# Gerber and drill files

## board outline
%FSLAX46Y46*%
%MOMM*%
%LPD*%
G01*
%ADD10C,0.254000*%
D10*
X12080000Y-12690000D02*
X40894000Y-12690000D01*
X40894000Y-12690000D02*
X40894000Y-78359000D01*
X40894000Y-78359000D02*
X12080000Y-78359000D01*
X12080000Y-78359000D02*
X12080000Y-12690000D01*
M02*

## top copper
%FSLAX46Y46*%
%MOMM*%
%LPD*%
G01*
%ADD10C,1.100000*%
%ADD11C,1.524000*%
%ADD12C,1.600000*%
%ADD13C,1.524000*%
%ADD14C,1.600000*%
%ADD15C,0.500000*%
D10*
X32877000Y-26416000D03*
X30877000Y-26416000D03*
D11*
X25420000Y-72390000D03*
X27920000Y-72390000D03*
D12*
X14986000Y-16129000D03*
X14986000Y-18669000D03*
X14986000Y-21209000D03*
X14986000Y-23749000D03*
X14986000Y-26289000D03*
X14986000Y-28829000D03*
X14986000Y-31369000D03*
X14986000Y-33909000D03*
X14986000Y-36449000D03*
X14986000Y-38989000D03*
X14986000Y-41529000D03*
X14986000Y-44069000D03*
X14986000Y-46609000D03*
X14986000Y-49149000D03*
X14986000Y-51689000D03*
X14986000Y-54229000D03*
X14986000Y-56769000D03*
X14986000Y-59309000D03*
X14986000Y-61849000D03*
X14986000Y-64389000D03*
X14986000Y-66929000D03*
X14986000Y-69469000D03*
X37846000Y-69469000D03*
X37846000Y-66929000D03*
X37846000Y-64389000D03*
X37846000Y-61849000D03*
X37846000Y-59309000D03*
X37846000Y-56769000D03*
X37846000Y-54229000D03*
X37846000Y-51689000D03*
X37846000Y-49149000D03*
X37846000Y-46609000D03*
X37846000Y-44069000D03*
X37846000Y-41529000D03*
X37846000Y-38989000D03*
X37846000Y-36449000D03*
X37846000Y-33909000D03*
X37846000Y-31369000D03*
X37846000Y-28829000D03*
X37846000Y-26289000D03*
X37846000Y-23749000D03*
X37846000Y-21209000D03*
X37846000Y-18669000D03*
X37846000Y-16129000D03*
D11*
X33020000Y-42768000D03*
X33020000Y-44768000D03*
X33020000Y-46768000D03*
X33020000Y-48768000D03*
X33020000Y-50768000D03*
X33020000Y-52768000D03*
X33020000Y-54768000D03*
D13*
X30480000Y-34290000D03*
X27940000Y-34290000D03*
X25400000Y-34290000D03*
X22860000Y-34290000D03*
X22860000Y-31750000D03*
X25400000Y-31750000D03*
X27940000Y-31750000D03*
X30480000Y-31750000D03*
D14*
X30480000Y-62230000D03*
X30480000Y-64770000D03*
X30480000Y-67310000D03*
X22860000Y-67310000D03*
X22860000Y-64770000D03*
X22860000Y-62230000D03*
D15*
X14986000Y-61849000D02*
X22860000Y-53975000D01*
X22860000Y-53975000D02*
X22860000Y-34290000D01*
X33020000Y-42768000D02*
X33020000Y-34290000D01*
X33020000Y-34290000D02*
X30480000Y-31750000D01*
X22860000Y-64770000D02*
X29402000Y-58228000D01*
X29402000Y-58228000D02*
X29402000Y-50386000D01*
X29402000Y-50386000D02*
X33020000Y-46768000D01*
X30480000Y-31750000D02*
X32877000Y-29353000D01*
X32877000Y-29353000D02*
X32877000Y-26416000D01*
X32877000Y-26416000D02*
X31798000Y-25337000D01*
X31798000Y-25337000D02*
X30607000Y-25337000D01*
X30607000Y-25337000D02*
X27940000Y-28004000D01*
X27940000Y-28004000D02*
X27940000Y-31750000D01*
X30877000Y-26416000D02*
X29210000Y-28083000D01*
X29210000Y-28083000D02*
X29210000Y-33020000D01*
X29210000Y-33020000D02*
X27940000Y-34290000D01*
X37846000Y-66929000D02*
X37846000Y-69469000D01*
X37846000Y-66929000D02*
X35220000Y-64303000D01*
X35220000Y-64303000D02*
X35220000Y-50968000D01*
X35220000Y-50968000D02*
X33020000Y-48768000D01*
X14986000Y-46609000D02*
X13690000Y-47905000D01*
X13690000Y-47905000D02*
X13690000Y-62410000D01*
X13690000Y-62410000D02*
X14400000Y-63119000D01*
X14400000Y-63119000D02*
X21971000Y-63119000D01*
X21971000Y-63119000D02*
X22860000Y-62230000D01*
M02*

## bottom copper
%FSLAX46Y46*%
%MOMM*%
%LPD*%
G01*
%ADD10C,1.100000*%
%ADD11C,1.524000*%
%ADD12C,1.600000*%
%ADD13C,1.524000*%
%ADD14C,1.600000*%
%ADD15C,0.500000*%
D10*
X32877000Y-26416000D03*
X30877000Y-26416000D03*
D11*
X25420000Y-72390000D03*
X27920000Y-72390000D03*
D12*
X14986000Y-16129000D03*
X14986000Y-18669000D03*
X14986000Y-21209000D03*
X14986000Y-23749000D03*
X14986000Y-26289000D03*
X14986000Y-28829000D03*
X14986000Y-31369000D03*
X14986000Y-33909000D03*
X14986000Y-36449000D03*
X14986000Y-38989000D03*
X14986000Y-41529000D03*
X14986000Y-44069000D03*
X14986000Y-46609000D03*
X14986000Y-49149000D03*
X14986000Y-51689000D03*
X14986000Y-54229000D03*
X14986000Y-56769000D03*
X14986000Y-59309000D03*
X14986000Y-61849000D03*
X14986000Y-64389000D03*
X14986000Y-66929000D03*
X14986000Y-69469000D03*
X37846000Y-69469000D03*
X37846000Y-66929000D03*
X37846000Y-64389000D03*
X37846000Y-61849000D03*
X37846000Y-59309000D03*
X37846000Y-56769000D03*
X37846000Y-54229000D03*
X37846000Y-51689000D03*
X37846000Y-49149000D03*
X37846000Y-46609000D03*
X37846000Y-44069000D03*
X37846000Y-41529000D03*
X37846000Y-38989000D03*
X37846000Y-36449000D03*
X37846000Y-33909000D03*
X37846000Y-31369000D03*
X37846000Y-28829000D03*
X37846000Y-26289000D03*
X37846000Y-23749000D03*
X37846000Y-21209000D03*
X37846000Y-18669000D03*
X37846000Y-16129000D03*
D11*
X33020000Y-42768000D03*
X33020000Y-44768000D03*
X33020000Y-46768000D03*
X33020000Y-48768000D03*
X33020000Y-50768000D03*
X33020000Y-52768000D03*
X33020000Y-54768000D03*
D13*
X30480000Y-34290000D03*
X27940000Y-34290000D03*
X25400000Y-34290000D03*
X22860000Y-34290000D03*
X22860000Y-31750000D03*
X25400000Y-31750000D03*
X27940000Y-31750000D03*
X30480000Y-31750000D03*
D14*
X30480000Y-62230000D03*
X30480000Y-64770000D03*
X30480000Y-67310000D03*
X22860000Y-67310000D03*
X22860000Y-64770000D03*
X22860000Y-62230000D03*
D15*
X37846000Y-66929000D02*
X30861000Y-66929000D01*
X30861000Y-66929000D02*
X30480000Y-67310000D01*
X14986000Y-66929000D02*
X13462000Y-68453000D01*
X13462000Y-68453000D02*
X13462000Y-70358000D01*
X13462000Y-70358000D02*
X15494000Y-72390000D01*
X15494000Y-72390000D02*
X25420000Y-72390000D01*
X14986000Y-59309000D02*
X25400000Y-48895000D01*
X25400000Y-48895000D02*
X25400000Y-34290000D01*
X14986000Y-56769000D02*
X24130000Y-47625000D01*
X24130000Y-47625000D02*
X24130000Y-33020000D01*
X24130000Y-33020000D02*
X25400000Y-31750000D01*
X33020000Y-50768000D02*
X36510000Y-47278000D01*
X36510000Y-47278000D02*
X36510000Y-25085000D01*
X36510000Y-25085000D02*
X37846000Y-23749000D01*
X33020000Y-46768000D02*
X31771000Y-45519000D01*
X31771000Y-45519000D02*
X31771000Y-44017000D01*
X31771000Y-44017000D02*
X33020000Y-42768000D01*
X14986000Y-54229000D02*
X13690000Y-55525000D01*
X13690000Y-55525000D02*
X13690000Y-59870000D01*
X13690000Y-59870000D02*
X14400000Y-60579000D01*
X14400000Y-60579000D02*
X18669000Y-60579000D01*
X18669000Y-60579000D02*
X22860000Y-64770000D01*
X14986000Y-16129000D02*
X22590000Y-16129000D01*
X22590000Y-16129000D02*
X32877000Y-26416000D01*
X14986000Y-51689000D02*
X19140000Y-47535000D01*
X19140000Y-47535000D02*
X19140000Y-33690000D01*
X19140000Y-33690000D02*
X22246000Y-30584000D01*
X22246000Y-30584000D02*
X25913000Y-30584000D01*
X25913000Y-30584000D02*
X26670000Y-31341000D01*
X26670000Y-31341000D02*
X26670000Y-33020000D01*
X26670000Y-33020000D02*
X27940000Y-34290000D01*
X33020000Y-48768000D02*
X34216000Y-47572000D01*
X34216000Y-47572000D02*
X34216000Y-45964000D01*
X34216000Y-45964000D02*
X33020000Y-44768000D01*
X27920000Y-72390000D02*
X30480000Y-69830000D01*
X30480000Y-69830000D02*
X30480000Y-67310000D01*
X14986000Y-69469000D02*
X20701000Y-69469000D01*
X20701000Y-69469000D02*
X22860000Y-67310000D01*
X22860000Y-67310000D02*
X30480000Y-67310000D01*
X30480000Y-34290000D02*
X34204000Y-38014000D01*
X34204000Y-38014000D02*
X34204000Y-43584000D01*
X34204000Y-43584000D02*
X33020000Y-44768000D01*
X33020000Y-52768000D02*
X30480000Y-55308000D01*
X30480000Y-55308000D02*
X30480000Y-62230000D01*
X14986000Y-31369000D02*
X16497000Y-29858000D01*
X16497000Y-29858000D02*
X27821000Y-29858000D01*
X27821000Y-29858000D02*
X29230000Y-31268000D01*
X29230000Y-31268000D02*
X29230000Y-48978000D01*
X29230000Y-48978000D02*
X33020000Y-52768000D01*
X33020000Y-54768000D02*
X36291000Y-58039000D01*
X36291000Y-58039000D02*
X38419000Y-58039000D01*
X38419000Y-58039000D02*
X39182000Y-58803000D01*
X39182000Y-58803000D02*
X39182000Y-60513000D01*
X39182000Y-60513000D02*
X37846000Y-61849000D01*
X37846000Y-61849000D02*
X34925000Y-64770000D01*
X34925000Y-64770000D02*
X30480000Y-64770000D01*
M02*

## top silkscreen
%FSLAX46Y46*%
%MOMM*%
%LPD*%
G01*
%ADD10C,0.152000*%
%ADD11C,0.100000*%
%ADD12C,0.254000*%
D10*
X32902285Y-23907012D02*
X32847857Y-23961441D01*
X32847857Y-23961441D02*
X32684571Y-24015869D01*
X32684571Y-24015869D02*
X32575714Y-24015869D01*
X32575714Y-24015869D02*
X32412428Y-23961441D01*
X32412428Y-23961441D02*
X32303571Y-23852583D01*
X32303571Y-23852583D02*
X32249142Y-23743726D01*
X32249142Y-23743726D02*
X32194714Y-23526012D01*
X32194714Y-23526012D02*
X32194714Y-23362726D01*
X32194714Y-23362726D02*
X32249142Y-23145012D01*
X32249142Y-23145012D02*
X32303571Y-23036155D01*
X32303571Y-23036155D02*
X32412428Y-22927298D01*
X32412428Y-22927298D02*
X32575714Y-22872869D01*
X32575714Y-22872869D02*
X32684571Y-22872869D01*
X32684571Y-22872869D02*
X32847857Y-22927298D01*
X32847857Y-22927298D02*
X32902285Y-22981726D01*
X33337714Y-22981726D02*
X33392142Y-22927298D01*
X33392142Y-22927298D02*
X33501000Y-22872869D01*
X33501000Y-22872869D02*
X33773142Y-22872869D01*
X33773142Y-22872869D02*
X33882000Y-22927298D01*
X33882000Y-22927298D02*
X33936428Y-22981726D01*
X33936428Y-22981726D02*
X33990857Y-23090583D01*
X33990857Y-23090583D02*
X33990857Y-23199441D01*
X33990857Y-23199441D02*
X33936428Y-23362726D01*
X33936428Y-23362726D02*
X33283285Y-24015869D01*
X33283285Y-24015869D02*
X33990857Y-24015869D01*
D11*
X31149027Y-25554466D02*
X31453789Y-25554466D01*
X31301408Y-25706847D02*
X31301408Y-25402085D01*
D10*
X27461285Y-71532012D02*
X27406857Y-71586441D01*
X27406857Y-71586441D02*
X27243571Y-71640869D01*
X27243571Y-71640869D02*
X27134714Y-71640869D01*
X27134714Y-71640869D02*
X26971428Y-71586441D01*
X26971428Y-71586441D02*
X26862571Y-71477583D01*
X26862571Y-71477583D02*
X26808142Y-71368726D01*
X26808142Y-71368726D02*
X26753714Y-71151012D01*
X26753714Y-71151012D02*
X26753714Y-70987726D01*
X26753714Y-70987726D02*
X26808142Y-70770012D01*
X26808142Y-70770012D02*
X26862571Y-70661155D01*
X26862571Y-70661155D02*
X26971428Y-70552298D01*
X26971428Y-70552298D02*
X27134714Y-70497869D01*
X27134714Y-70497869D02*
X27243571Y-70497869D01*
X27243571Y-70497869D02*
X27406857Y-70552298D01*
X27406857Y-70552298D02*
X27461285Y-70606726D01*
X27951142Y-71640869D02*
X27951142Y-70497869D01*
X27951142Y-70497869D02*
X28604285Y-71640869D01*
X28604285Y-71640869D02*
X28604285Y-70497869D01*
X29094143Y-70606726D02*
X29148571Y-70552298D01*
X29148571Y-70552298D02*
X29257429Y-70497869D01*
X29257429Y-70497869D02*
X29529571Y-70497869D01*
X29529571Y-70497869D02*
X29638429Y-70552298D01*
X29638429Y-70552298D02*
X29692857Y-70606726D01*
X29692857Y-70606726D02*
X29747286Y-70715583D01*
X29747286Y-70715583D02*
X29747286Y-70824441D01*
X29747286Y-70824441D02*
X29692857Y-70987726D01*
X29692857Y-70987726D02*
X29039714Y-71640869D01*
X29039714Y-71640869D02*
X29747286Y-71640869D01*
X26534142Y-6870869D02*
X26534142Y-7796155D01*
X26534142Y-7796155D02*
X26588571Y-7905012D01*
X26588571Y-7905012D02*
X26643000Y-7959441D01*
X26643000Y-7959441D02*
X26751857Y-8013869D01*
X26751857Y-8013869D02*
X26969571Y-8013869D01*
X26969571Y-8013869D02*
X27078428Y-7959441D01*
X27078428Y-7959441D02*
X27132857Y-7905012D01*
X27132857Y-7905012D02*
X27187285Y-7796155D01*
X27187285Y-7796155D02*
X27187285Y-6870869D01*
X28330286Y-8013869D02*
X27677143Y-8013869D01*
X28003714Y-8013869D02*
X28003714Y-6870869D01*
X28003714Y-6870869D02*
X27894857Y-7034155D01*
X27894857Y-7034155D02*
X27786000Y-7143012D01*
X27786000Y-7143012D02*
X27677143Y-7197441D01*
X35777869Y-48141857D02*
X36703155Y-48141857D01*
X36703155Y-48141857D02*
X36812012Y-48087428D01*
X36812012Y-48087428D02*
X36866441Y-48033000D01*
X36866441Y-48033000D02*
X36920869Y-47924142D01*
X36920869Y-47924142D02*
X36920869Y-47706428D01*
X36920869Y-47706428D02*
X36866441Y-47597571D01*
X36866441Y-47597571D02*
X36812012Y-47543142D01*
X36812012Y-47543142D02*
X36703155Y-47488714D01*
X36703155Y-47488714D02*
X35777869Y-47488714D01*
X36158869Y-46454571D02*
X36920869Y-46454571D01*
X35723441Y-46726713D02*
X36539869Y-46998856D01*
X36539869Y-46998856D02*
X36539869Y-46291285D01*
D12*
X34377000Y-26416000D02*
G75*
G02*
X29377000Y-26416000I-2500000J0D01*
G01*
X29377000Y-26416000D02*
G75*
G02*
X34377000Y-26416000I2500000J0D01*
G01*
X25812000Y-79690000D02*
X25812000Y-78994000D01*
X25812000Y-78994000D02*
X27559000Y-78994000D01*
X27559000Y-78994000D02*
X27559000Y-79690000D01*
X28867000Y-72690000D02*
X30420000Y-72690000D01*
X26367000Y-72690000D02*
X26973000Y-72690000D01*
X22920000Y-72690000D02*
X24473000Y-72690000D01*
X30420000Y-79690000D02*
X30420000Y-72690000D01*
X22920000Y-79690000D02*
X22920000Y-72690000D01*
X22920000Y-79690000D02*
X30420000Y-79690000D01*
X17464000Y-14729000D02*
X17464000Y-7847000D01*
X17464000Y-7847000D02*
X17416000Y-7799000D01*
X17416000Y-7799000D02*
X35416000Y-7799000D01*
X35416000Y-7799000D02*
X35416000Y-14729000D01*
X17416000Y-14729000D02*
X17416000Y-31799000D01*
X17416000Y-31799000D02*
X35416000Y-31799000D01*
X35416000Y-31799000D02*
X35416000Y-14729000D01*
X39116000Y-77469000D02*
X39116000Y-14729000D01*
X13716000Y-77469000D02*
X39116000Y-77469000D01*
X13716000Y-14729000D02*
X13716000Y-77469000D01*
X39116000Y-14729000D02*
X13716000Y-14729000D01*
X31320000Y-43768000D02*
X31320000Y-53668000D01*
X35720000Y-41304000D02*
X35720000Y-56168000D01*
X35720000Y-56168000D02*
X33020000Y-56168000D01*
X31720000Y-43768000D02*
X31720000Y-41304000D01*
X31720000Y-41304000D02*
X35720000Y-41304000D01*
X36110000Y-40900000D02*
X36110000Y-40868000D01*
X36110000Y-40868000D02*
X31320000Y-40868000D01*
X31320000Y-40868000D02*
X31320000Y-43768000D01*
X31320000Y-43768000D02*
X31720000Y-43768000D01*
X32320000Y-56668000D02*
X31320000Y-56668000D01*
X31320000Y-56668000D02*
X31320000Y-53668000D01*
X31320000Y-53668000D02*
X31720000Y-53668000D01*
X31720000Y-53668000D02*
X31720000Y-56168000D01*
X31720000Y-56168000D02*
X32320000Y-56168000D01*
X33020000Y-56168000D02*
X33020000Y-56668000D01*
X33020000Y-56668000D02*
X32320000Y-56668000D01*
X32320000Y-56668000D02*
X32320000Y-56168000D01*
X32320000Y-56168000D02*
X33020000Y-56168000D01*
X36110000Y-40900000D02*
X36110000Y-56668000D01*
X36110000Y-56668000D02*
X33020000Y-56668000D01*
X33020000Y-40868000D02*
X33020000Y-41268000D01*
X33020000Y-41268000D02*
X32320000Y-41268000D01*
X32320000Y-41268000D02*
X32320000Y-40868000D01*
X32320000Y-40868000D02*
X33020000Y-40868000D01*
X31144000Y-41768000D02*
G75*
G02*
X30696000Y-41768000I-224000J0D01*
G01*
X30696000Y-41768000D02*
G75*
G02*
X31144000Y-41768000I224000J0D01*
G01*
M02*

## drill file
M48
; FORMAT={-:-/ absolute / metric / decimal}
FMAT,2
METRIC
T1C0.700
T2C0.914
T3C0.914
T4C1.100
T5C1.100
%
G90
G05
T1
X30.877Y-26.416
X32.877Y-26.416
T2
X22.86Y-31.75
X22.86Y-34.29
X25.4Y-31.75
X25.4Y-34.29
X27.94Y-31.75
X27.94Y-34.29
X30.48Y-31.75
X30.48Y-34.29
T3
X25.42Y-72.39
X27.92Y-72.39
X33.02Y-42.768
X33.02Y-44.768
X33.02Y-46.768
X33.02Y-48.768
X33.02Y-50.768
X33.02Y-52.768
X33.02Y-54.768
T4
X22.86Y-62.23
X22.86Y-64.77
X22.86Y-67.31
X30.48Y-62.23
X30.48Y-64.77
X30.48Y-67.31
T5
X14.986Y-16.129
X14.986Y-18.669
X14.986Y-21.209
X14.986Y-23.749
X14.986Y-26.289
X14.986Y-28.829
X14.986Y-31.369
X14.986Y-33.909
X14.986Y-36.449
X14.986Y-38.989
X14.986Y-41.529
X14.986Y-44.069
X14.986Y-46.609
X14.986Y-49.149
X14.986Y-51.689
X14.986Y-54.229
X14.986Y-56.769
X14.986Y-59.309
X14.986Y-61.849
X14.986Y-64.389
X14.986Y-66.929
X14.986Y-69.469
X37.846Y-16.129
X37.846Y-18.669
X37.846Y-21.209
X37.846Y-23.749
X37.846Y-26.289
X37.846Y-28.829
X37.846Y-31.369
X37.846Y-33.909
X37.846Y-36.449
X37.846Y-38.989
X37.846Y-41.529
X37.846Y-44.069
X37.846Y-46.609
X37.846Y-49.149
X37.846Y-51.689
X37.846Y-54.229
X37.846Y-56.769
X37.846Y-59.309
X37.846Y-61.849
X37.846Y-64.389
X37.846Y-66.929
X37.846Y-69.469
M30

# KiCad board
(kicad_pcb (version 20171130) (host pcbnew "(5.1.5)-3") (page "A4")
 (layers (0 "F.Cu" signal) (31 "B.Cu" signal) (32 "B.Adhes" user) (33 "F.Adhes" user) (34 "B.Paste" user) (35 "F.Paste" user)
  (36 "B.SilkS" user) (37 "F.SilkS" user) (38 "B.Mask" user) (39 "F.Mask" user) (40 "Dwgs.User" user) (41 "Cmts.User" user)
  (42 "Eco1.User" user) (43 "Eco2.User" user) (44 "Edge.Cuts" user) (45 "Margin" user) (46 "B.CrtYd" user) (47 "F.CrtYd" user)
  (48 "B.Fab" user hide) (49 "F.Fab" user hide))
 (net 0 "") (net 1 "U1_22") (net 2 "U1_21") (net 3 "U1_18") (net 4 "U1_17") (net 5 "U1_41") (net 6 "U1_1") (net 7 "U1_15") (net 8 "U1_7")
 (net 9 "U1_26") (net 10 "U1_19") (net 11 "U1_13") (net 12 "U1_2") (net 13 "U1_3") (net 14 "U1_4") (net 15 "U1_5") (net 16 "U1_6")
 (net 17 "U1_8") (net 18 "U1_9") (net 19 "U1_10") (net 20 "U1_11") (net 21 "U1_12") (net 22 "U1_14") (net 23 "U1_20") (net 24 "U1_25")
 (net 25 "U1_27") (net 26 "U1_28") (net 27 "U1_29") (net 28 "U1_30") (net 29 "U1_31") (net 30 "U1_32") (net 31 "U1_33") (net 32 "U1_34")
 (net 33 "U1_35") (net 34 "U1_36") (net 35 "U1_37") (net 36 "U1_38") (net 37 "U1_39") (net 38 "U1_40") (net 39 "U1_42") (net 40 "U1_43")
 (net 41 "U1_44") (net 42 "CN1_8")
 (segment (start 37.846 66.929) (end 30.861 66.929) (width 0.5) (layer "B.Cu") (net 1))
 (segment (start 30.861 66.929) (end 30.48 67.31) (width 0.5) (layer "B.Cu") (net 1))
 (segment (start 14.986 66.929) (end 13.462 68.453) (width 0.5) (layer "B.Cu") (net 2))
 (segment (start 13.462 68.453) (end 13.462 70.358) (width 0.5) (layer "B.Cu") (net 2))
 (segment (start 13.462 70.358) (end 15.494 72.39) (width 0.5) (layer "B.Cu") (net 2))
 (segment (start 15.494 72.39) (end 25.42 72.39) (width 0.5) (layer "B.Cu") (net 2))
 (segment (start 14.986 59.309) (end 25.4 48.895) (width 0.5) (layer "B.Cu") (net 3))
 (segment (start 25.4 48.895) (end 25.4 34.29) (width 0.5) (layer "B.Cu") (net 3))
 (segment (start 14.986 56.769) (end 24.13 47.625) (width 0.5) (layer "B.Cu") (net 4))
 (segment (start 24.13 47.625) (end 24.13 33.02) (width 0.5) (layer "B.Cu") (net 4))
 (segment (start 24.13 33.02) (end 25.4 31.75) (width 0.5) (layer "B.Cu") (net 4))
 (segment (start 33.02 50.768) (end 36.51 47.278) (width 0.5) (layer "B.Cu") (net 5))
 (segment (start 36.51 47.278) (end 36.51 25.085) (width 0.5) (layer "B.Cu") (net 5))
 (segment (start 36.51 25.085) (end 37.846 23.749) (width 0.5) (layer "B.Cu") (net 5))
 (segment (start 33.02 46.768) (end 31.771 45.519) (width 0.5) (layer "B.Cu") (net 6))
 (segment (start 31.771 45.519) (end 31.771 44.017) (width 0.5) (layer "B.Cu") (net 6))
 (segment (start 31.771 44.017) (end 33.02 42.768) (width 0.5) (layer "B.Cu") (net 6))
 (segment (start 14.986 54.229) (end 13.69 55.525) (width 0.5) (layer "B.Cu") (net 6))
 (segment (start 13.69 55.525) (end 13.69 59.87) (width 0.5) (layer "B.Cu") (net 6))
 (segment (start 13.69 59.87) (end 14.4 60.579) (width 0.5) (layer "B.Cu") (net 6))
 (segment (start 14.4 60.579) (end 18.669 60.579) (width 0.5) (layer "B.Cu") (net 6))
 (segment (start 18.669 60.579) (end 22.86 64.77) (width 0.5) (layer "B.Cu") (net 6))
 (segment (start 14.986 16.129) (end 22.59 16.129) (width 0.5) (layer "B.Cu") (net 6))
 (segment (start 22.59 16.129) (end 32.877 26.416) (width 0.5) (layer "B.Cu") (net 6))
 (segment (start 14.986 51.689) (end 19.14 47.535) (width 0.5) (layer "B.Cu") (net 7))
 (segment (start 19.14 47.535) (end 19.14 33.69) (width 0.5) (layer "B.Cu") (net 7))
 (segment (start 19.14 33.69) (end 22.246 30.584) (width 0.5) (layer "B.Cu") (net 7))
 (segment (start 22.246 30.584) (end 25.913 30.584) (width 0.5) (layer "B.Cu") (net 7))
 (segment (start 25.913 30.584) (end 26.67 31.341) (width 0.5) (layer "B.Cu") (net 7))
 (segment (start 26.67 31.341) (end 26.67 33.02) (width 0.5) (layer "B.Cu") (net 7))
 (segment (start 26.67 33.02) (end 27.94 34.29) (width 0.5) (layer "B.Cu") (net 7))
 (segment (start 33.02 48.768) (end 34.216 47.572) (width 0.5) (layer "B.Cu") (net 1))
 (segment (start 34.216 47.572) (end 34.216 45.964) (width 0.5) (layer "B.Cu") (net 1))
 (segment (start 34.216 45.964) (end 33.02 44.768) (width 0.5) (layer "B.Cu") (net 1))
 (segment (start 27.92 72.39) (end 30.48 69.83) (width 0.5) (layer "B.Cu") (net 1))
 (segment (start 30.48 69.83) (end 30.48 67.31) (width 0.5) (layer "B.Cu") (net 1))
 (segment (start 14.986 69.469) (end 20.701 69.469) (width 0.5) (layer "B.Cu") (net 1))
 (segment (start 20.701 69.469) (end 22.86 67.31) (width 0.5) (layer "B.Cu") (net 1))
 (segment (start 22.86 67.31) (end 30.48 67.31) (width 0.5) (layer "B.Cu") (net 1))
 (segment (start 30.48 34.29) (end 34.204 38.014) (width 0.5) (layer "B.Cu") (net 1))
 (segment (start 34.204 38.014) (end 34.204 43.584) (width 0.5) (layer "B.Cu") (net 1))
 (segment (start 34.204 43.584) (end 33.02 44.768) (width 0.5) (layer "B.Cu") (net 1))
 (segment (start 33.02 52.768) (end 30.48 55.308) (width 0.5) (layer "B.Cu") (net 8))
 (segment (start 30.48 55.308) (end 30.48 62.23) (width 0.5) (layer "B.Cu") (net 8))
 (segment (start 14.986 31.369) (end 16.497 29.858) (width 0.5) (layer "B.Cu") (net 8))
 (segment (start 16.497 29.858) (end 27.821 29.858) (width 0.5) (layer "B.Cu") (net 8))
 (segment (start 27.821 29.858) (end 29.23 31.268) (width 0.5) (layer "B.Cu") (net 8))
 (segment (start 29.23 31.268) (end 29.23 48.978) (width 0.5) (layer "B.Cu") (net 8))
 (segment (start 29.23 48.978) (end 33.02 52.768) (width 0.5) (layer "B.Cu") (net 8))
 (segment (start 33.02 54.768) (end 36.291 58.039) (width 0.5) (layer "B.Cu") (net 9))
 (segment (start 36.291 58.039) (end 38.419 58.039) (width 0.5) (layer "B.Cu") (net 9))
 (segment (start 38.419 58.039) (end 39.182 58.803) (width 0.5) (layer "B.Cu") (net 9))
 (segment (start 39.182 58.803) (end 39.182 60.513) (width 0.5) (layer "B.Cu") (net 9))
 (segment (start 39.182 60.513) (end 37.846 61.849) (width 0.5) (layer "B.Cu") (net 9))
 (segment (start 37.846 61.849) (end 34.925 64.77) (width 0.5) (layer "B.Cu") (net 9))
 (segment (start 34.925 64.77) (end 30.48 64.77) (width 0.5) (layer "B.Cu") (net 9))
 (gr_line (start 12.08 12.69) (end 40.894 12.69) (width 0.254) (layer "Edge.Cuts"))
 (gr_line (start 40.894 12.69) (end 40.894 78.359) (width 0.254) (layer "Edge.Cuts"))
 (gr_line (start 40.894 78.359) (end 12.08 78.359) (width 0.254) (layer "Edge.Cuts"))
 (gr_line (start 12.08 78.359) (end 12.08 12.69) (width 0.254) (layer "Edge.Cuts"))
 (segment (start 14.986 61.849) (end 22.86 53.975) (width 0.5) (layer "F.Cu") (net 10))
 (segment (start 22.86 53.975) (end 22.86 34.29) (width 0.5) (layer "F.Cu") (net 10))
 (segment (start 33.02 42.768) (end 33.02 34.29) (width 0.5) (layer "F.Cu") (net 6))
 (segment (start 33.02 34.29) (end 30.48 31.75) (width 0.5) (layer "F.Cu") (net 6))
 (segment (start 22.86 64.77) (end 29.402 58.228) (width 0.5) (layer "F.Cu") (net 6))
 (segment (start 29.402 58.228) (end 29.402 50.386) (width 0.5) (layer "F.Cu") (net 6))
 (segment (start 29.402 50.386) (end 33.02 46.768) (width 0.5) (layer "F.Cu") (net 6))
 (segment (start 30.48 31.75) (end 32.877 29.353) (width 0.5) (layer "F.Cu") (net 6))
 (segment (start 32.877 29.353) (end 32.877 26.416) (width 0.5) (layer "F.Cu") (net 6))
 (segment (start 32.877 26.416) (end 31.798 25.337) (width 0.5) (layer "F.Cu") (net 6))
 (segment (start 31.798 25.337) (end 30.607 25.337) (width 0.5) (layer "F.Cu") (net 6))
 (segment (start 30.607 25.337) (end 27.94 28.004) (width 0.5) (layer "F.Cu") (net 6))
 (segment (start 27.94 28.004) (end 27.94 31.75) (width 0.5) (layer "F.Cu") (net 6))
 (segment (start 30.877 26.416) (end 29.21 28.083) (width 0.5) (layer "F.Cu") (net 7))
 (segment (start 29.21 28.083) (end 29.21 33.02) (width 0.5) (layer "F.Cu") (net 7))
 (segment (start 29.21 33.02) (end 27.94 34.29) (width 0.5) (layer "F.Cu") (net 7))
 (segment (start 37.846 66.929) (end 37.846 69.469) (width 0.5) (layer "F.Cu") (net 1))
 (segment (start 37.846 66.929) (end 35.22 64.303) (width 0.5) (layer "F.Cu") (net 1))
 (segment (start 35.22 64.303) (end 35.22 50.968) (width 0.5) (layer "F.Cu") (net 1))
 (segment (start 35.22 50.968) (end 33.02 48.768) (width 0.5) (layer "F.Cu") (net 1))
 (segment (start 14.986 46.609) (end 13.69 47.905) (width 0.5) (layer "F.Cu") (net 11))
 (segment (start 13.69 47.905) (end 13.69 62.41) (width 0.5) (layer "F.Cu") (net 11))
 (segment (start 13.69 62.41) (end 14.4 63.119) (width 0.5) (layer "F.Cu") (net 11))
 (segment (start 14.4 63.119) (end 21.971 63.119) (width 0.5) (layer "F.Cu") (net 11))
 (segment (start 21.971 63.119) (end 22.86 62.23) (width 0.5) (layer "F.Cu") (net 11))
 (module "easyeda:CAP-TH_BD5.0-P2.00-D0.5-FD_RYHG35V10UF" (layer "F.Cu") (at 31.877 26.416 0)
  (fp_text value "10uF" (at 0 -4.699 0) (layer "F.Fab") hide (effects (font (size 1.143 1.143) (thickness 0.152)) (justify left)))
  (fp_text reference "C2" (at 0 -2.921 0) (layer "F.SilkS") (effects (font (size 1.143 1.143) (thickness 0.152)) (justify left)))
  (fp_circle (center 0 0) (end 2.5 0) (layer "F.SilkS") (width 0.254))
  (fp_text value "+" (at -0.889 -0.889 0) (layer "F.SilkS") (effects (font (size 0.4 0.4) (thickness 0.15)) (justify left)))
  (pad 2 thru_hole circle (at 1 0 0) (size 1.1 1.1) (layers "*.Cu" "*.Paste" "*.Mask") (drill 0.7) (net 6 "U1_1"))
  (pad 1 thru_hole circle (at -1 0 0) (size 1.1 1.1) (layers "*.Cu" "*.Paste" "*.Mask") (drill 0.7) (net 7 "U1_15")))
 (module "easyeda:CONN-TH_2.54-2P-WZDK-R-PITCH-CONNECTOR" (layer "F.Cu") (at 26.67 72.39 0)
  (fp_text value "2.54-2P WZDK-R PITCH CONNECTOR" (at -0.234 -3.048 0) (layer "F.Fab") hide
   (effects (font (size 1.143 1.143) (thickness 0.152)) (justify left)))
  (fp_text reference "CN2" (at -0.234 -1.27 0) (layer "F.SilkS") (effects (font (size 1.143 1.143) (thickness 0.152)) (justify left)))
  (fp_line (start -0.858 7.3) (end -0.858 6.604) (width 0.254) (layer "F.SilkS"))
  (fp_line (start -0.858 6.604) (end 0.889 6.604) (width 0.254) (layer "F.SilkS"))
  (fp_line (start 0.889 6.604) (end 0.889 7.3) (width 0.254) (layer "F.SilkS"))
  (fp_line (start 2.197 0.3) (end 3.75 0.3) (width 0.254) (layer "F.SilkS"))
  (fp_line (start -0.303 0.3) (end 0.303 0.3) (width 0.254) (layer "F.SilkS"))
  (fp_line (start -3.75 0.3) (end -2.197 0.3) (width 0.254) (layer "F.SilkS"))
  (fp_line (start 3.75 7.3) (end 3.75 0.3) (width 0.254) (layer "F.SilkS"))
  (fp_line (start -3.75 7.3) (end -3.75 0.3) (width 0.254) (layer "F.SilkS"))
  (fp_line (start -3.75 7.3) (end 3.75 7.3) (width 0.254) (layer "F.SilkS"))
  (pad 1 thru_hole circle (at -1.25 0 0) (size 1.524 1.524) (layers "*.Cu" "*.Paste" "*.Mask") (drill 0.914) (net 2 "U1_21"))
  (pad 2 thru_hole circle (at 1.25 0 0) (size 1.524 1.524) (layers "*.Cu" "*.Paste" "*.Mask") (drill 0.914) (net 1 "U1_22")))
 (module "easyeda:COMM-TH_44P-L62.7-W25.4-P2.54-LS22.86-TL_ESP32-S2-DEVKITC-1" (layer "F.Cu") (at 26.416 42.799)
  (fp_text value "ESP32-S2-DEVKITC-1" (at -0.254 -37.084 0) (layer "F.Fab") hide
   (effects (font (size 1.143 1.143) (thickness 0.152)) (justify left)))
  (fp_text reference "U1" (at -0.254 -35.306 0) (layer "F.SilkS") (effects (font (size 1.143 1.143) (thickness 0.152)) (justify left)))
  (fp_line (start -8.952 -28.07) (end -8.952 -34.952) (width 0.254) (layer "F.SilkS"))
  (fp_line (start -8.952 -34.952) (end -9 -35) (width 0.254) (layer "F.SilkS"))
  (fp_line (start -9 -35) (end 9 -35) (width 0.254) (layer "F.SilkS"))
  (fp_line (start 9 -35) (end 9 -28.07) (width 0.254) (layer "F.SilkS"))
  (fp_line (start -9 -28.07) (end -9 -11) (width 0.254) (layer "F.SilkS"))
  (fp_line (start -9 -11) (end 9 -11) (width 0.254) (layer "F.SilkS"))
  (fp_line (start 9 -11) (end 9 -28.07) (width 0.254) (layer "F.SilkS"))
  (fp_line (start 12.7 34.67) (end 12.7 -28.07) (width 0.254) (layer "F.SilkS"))
  (fp_line (start -12.7 34.67) (end 12.7 34.67) (width 0.254) (layer "F.SilkS"))
  (fp_line (start -12.7 -28.07) (end -12.7 34.67) (width 0.254) (layer "F.SilkS"))
  (fp_line (start 12.7 -28.07) (end -12.7 -28.07) (width 0.254) (layer "F.SilkS"))
  (pad 1 thru_hole circle (at -11.43 -26.67 0) (size 1.6 1.6) (layers "*.Cu" "*.Paste" "*.Mask") (drill 1.1) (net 6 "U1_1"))
  (pad 2 thru_hole circle (at -11.43 -24.13 0) (size 1.6 1.6) (layers "*.Cu" "*.Paste" "*.Mask") (drill 1.1) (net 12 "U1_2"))
  (pad 3 thru_hole circle (at -11.43 -21.59 0) (size 1.6 1.6) (layers "*.Cu" "*.Paste" "*.Mask") (drill 1.1) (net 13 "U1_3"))
  (pad 4 thru_hole circle (at -11.43 -19.05 0) (size 1.6 1.6) (layers "*.Cu" "*.Paste" "*.Mask") (drill 1.1) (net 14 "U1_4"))
  (pad 5 thru_hole circle (at -11.43 -16.51 0) (size 1.6 1.6) (layers "*.Cu" "*.Paste" "*.Mask") (drill 1.1) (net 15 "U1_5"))
  (pad 6 thru_hole circle (at -11.43 -13.97 0) (size 1.6 1.6) (layers "*.Cu" "*.Paste" "*.Mask") (drill 1.1) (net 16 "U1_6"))
  (pad 7 thru_hole circle (at -11.43 -11.43 0) (size 1.6 1.6) (layers "*.Cu" "*.Paste" "*.Mask") (drill 1.1) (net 8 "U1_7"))
  (pad 8 thru_hole circle (at -11.43 -8.89 0) (size 1.6 1.6) (layers "*.Cu" "*.Paste" "*.Mask") (drill 1.1) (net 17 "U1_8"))
  (pad 9 thru_hole circle (at -11.43 -6.35 0) (size 1.6 1.6) (layers "*.Cu" "*.Paste" "*.Mask") (drill 1.1) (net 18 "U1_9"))
  (pad 10 thru_hole circle (at -11.43 -3.81 0) (size 1.6 1.6) (layers "*.Cu" "*.Paste" "*.Mask") (drill 1.1) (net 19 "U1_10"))
  (pad 11 thru_hole circle (at -11.43 -1.27 0) (size 1.6 1.6) (layers "*.Cu" "*.Paste" "*.Mask") (drill 1.1) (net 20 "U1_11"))
  (pad 12 thru_hole circle (at -11.43 1.27 0) (size 1.6 1.6) (layers "*.Cu" "*.Paste" "*.Mask") (drill 1.1) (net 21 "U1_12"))
  (pad 13 thru_hole circle (at -11.43 3.81 0) (size 1.6 1.6) (layers "*.Cu" "*.Paste" "*.Mask") (drill 1.1) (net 11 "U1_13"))
  (pad 14 thru_hole circle (at -11.43 6.35 0) (size 1.6 1.6) (layers "*.Cu" "*.Paste" "*.Mask") (drill 1.1) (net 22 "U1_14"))
  (pad 15 thru_hole circle (at -11.43 8.89 0) (size 1.6 1.6) (layers "*.Cu" "*.Paste" "*.Mask") (drill 1.1) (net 7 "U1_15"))
  (pad 16 thru_hole circle (at -11.43 11.43 0) (size 1.6 1.6) (layers "*.Cu" "*.Paste" "*.Mask") (drill 1.1) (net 6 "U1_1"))
  (pad 17 thru_hole circle (at -11.43 13.97 0) (size 1.6 1.6) (layers "*.Cu" "*.Paste" "*.Mask") (drill 1.1) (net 4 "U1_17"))
  (pad 18 thru_hole circle (at -11.43 16.51 0) (size 1.6 1.6) (layers "*.Cu" "*.Paste" "*.Mask") (drill 1.1) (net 3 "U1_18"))
  (pad 19 thru_hole circle (at -11.43 19.05 0) (size 1.6 1.6) (layers "*.Cu" "*.Paste" "*.Mask") (drill 1.1) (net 10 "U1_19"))
  (pad 20 thru_hole circle (at -11.43 21.59 0) (size 1.6 1.6) (layers "*.Cu" "*.Paste" "*.Mask") (drill 1.1) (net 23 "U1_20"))
  (pad 21 thru_hole circle (at -11.43 24.13 0) (size 1.6 1.6) (layers "*.Cu" "*.Paste" "*.Mask") (drill 1.1) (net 2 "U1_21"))
  (pad 22 thru_hole circle (at -11.43 26.67 0) (size 1.6 1.6) (layers "*.Cu" "*.Paste" "*.Mask") (drill 1.1) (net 1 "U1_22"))
  (pad 23 thru_hole circle (at 11.43 26.67 0) (size 1.6 1.6) (layers "*.Cu" "*.Paste" "*.Mask") (drill 1.1) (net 1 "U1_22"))
  (pad 24 thru_hole circle (at 11.43 24.13 0) (size 1.6 1.6) (layers "*.Cu" "*.Paste" "*.Mask") (drill 1.1) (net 1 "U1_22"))
  (pad 25 thru_hole circle (at 11.43 21.59 0) (size 1.6 1.6) (layers "*.Cu" "*.Paste" "*.Mask") (drill 1.1) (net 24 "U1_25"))
  (pad 26 thru_hole circle (at 11.43 19.05 0) (size 1.6 1.6) (layers "*.Cu" "*.Paste" "*.Mask") (drill 1.1) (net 9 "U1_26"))
  (pad 27 thru_hole circle (at 11.43 16.51 0) (size 1.6 1.6) (layers "*.Cu" "*.Paste" "*.Mask") (drill 1.1) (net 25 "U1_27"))
  (pad 28 thru_hole circle (at 11.43 13.97 0) (size 1.6 1.6) (layers "*.Cu" "*.Paste" "*.Mask") (drill 1.1) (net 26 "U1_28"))
  (pad 29 thru_hole circle (at 11.43 11.43 0) (size 1.6 1.6) (layers "*.Cu" "*.Paste" "*.Mask") (drill 1.1) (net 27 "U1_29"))
  (pad 30 thru_hole circle (at 11.43 8.89 0) (size 1.6 1.6) (layers "*.Cu" "*.Paste" "*.Mask") (drill 1.1) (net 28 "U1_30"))
  (pad 31 thru_hole circle (at 11.43 6.35 0) (size 1.6 1.6) (layers "*.Cu" "*.Paste" "*.Mask") (drill 1.1) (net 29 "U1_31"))
  (pad 32 thru_hole circle (at 11.43 3.81 0) (size 1.6 1.6) (layers "*.Cu" "*.Paste" "*.Mask") (drill 1.1) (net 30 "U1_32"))
  (pad 33 thru_hole circle (at 11.43 1.27 0) (size 1.6 1.6) (layers "*.Cu" "*.Paste" "*.Mask") (drill 1.1) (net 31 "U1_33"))
  (pad 34 thru_hole circle (at 11.43 -1.27 0) (size 1.6 1.6) (layers "*.Cu" "*.Paste" "*.Mask") (drill 1.1) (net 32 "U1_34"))
  (pad 35 thru_hole circle (at 11.43 -3.81 0) (size 1.6 1.6) (layers "*.Cu" "*.Paste" "*.Mask") (drill 1.1) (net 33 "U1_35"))
  (pad 36 thru_hole circle (at 11.43 -6.35 0) (size 1.6 1.6) (layers "*.Cu" "*.Paste" "*.Mask") (drill 1.1) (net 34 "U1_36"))
  (pad 37 thru_hole circle (at 11.43 -8.89 0) (size 1.6 1.6) (layers "*.Cu" "*.Paste" "*.Mask") (drill 1.1) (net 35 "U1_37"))
  (pad 38 thru_hole circle (at 11.43 -11.43 0) (size 1.6 1.6) (layers "*.Cu" "*.Paste" "*.Mask") (drill 1.1) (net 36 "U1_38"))
  (pad 39 thru_hole circle (at 11.43 -13.97 0) (size 1.6 1.6) (layers "*.Cu" "*.Paste" "*.Mask") (drill 1.1) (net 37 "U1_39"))
  (pad 40 thru_hole circle (at 11.43 -16.51 0) (size 1.6 1.6) (layers "*.Cu" "*.Paste" "*.Mask") (drill 1.1) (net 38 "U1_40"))
  (pad 41 thru_hole circle (at 11.43 -19.05 0) (size 1.6 1.6) (layers "*.Cu" "*.Paste" "*.Mask") (drill 1.1) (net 5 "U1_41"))
  (pad 42 thru_hole circle (at 11.43 -21.59 0) (size 1.6 1.6) (layers "*.Cu" "*.Paste" "*.Mask") (drill 1.1) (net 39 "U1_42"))
  (pad 43 thru_hole circle (at 11.43 -24.13 0) (size 1.6 1.6) (layers "*.Cu" "*.Paste" "*.Mask") (drill 1.1) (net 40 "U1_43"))
  (pad 44 thru_hole circle (at 11.43 -26.67 0) (size 1.6 1.6) (layers "*.Cu" "*.Paste" "*.Mask") (drill 1.1) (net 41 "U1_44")))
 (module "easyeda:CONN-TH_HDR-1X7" (layer "F.Cu") (at 33.02 48.768 -90)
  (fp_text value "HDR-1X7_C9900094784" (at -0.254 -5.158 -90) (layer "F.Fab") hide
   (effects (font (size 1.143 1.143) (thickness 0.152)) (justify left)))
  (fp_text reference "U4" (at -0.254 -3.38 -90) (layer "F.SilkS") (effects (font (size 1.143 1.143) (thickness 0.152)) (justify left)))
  (fp_line (start -5 1.7) (end 4.9 1.7) (width 0.254) (layer "F.SilkS"))
  (fp_line (start -7.464 -2.7) (end 7.4 -2.7) (width 0.254) (layer "F.SilkS"))
  (fp_line (start 7.4 -2.7) (end 7.4 0) (width 0.254) (layer "F.SilkS"))
  (fp_line (start -5 1.3) (end -7.464 1.3) (width 0.254) (layer "F.SilkS"))
  (fp_line (start -7.464 1.3) (end -7.464 -2.7) (width 0.254) (layer "F.SilkS"))
  (fp_line (start -7.868 -3.09) (end -7.9 -3.09) (width 0.254) (layer "F.SilkS"))
  (fp_line (start -7.9 -3.09) (end -7.9 1.7) (width 0.254) (layer "F.SilkS"))
  (fp_line (start -7.9 1.7) (end -5 1.7) (width 0.254) (layer "F.SilkS"))
  (fp_line (start -5 1.7) (end -5 1.3) (width 0.254) (layer "F.SilkS"))
  (fp_line (start 7.9 0.7) (end 7.9 1.7) (width 0.254) (layer "F.SilkS"))
  (fp_line (start 7.9 1.7) (end 4.9 1.7) (width 0.254) (layer "F.SilkS"))
  (fp_line (start 4.9 1.7) (end 4.9 1.3) (width 0.254) (layer "F.SilkS"))
  (fp_line (start 4.9 1.3) (end 7.4 1.3) (width 0.254) (layer "F.SilkS"))
  (fp_line (start 7.4 1.3) (end 7.4 0.7) (width 0.254) (layer "F.SilkS"))
  (fp_line (start 7.4 0) (end 7.9 0) (width 0.254) (layer "F.SilkS"))
  (fp_line (start 7.9 0) (end 7.9 0.7) (width 0.254) (layer "F.SilkS"))
  (fp_line (start 7.9 0.7) (end 7.4 0.7) (width 0.254) (layer "F.SilkS"))
  (fp_line (start 7.4 0.7) (end 7.4 0) (width 0.254) (layer "F.SilkS"))
  (fp_line (start -7.868 -3.09) (end 7.9 -3.09) (width 0.254) (layer "F.SilkS"))
  (fp_line (start 7.9 -3.09) (end 7.9 0) (width 0.254) (layer "F.SilkS"))
  (fp_line (start -7.9 0) (end -7.5 0) (width 0.254) (layer "F.SilkS"))
  (fp_line (start -7.5 0) (end -7.5 0.7) (width 0.254) (layer "F.SilkS"))
  (fp_line (start -7.5 0.7) (end -7.9 0.7) (width 0.254) (layer "F.SilkS"))
  (fp_line (start -7.9 0.7) (end -7.9 0) (width 0.254) (layer "F.SilkS"))
  (fp_circle (center -7 2.1) (end -6.776 2.1) (layer "F.SilkS") (width 0.254))
  (pad 1 thru_hole circle (at -6 0 -90) (size 1.524 1.524) (layers "*.Cu" "*.Paste" "*.Mask") (drill 0.914) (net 6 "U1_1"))
  (pad 2 thru_hole circle (at -4 0 -90) (size 1.524 1.524) (layers "*.Cu" "*.Paste" "*.Mask") (drill 0.914) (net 1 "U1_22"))
  (pad 3 thru_hole circle (at -2 0 -90) (size 1.524 1.524) (layers "*.Cu" "*.Paste" "*.Mask") (drill 0.914) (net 6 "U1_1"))
  (pad 4 thru_hole circle (at 0 0 -90) (size 1.524 1.524) (layers "*.Cu" "*.Paste" "*.Mask") (drill 0.914) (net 1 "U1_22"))
  (pad 5 thru_hole circle (at 2 0 -90) (size 1.524 1.524) (layers "*.Cu" "*.Paste" "*.Mask") (drill 0.914) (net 5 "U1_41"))
  (pad 6 thru_hole circle (at 4 0 -90) (size 1.524 1.524) (layers "*.Cu" "*.Paste" "*.Mask") (drill 0.914) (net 8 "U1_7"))
  (pad 7 thru_hole circle (at 6 0 -90) (size 1.524 1.524) (layers "*.Cu" "*.Paste" "*.Mask") (drill 0.914) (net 9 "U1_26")))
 (via (at 30.48 34.29) (size 1.524) (drill 0.914) (layers "F.Cu" "B.Cu") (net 1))
 (via (at 27.94 34.29) (size 1.524) (drill 0.914) (layers "F.Cu" "B.Cu") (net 7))
 (via (at 25.4 34.29) (size 1.524) (drill 0.914) (layers "F.Cu" "B.Cu") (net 3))
 (via (at 22.86 34.29) (size 1.524) (drill 0.914) (layers "F.Cu" "B.Cu") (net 10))
 (via (at 22.86 31.75) (size 1.524) (drill 0.914) (layers "F.Cu" "B.Cu") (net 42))
 (via (at 25.4 31.75) (size 1.524) (drill 0.914) (layers "F.Cu" "B.Cu") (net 4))
 (via (at 27.94 31.75) (size 1.524) (drill 0.914) (layers "F.Cu" "B.Cu") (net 6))
 (via (at 30.48 31.75) (size 1.524) (drill 0.914) (layers "F.Cu" "B.Cu") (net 6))
 (via (at 30.48 62.23) (size 1.6) (drill 1.1) (layers "F.Cu" "B.Cu") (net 8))
 (via (at 30.48 64.77) (size 1.6) (drill 1.1) (layers "F.Cu" "B.Cu") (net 9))
 (via (at 30.48 67.31) (size 1.6) (drill 1.1) (layers "F.Cu" "B.Cu") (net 1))
 (via (at 22.86 67.31) (size 1.6) (drill 1.1) (layers "F.Cu" "B.Cu") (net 1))
 (via (at 22.86 64.77) (size 1.6) (drill 1.1) (layers "F.Cu" "B.Cu") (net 6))
 (via (at 22.86 62.23) (size 1.6) (drill 1.1) (layers "F.Cu" "B.Cu") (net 11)))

